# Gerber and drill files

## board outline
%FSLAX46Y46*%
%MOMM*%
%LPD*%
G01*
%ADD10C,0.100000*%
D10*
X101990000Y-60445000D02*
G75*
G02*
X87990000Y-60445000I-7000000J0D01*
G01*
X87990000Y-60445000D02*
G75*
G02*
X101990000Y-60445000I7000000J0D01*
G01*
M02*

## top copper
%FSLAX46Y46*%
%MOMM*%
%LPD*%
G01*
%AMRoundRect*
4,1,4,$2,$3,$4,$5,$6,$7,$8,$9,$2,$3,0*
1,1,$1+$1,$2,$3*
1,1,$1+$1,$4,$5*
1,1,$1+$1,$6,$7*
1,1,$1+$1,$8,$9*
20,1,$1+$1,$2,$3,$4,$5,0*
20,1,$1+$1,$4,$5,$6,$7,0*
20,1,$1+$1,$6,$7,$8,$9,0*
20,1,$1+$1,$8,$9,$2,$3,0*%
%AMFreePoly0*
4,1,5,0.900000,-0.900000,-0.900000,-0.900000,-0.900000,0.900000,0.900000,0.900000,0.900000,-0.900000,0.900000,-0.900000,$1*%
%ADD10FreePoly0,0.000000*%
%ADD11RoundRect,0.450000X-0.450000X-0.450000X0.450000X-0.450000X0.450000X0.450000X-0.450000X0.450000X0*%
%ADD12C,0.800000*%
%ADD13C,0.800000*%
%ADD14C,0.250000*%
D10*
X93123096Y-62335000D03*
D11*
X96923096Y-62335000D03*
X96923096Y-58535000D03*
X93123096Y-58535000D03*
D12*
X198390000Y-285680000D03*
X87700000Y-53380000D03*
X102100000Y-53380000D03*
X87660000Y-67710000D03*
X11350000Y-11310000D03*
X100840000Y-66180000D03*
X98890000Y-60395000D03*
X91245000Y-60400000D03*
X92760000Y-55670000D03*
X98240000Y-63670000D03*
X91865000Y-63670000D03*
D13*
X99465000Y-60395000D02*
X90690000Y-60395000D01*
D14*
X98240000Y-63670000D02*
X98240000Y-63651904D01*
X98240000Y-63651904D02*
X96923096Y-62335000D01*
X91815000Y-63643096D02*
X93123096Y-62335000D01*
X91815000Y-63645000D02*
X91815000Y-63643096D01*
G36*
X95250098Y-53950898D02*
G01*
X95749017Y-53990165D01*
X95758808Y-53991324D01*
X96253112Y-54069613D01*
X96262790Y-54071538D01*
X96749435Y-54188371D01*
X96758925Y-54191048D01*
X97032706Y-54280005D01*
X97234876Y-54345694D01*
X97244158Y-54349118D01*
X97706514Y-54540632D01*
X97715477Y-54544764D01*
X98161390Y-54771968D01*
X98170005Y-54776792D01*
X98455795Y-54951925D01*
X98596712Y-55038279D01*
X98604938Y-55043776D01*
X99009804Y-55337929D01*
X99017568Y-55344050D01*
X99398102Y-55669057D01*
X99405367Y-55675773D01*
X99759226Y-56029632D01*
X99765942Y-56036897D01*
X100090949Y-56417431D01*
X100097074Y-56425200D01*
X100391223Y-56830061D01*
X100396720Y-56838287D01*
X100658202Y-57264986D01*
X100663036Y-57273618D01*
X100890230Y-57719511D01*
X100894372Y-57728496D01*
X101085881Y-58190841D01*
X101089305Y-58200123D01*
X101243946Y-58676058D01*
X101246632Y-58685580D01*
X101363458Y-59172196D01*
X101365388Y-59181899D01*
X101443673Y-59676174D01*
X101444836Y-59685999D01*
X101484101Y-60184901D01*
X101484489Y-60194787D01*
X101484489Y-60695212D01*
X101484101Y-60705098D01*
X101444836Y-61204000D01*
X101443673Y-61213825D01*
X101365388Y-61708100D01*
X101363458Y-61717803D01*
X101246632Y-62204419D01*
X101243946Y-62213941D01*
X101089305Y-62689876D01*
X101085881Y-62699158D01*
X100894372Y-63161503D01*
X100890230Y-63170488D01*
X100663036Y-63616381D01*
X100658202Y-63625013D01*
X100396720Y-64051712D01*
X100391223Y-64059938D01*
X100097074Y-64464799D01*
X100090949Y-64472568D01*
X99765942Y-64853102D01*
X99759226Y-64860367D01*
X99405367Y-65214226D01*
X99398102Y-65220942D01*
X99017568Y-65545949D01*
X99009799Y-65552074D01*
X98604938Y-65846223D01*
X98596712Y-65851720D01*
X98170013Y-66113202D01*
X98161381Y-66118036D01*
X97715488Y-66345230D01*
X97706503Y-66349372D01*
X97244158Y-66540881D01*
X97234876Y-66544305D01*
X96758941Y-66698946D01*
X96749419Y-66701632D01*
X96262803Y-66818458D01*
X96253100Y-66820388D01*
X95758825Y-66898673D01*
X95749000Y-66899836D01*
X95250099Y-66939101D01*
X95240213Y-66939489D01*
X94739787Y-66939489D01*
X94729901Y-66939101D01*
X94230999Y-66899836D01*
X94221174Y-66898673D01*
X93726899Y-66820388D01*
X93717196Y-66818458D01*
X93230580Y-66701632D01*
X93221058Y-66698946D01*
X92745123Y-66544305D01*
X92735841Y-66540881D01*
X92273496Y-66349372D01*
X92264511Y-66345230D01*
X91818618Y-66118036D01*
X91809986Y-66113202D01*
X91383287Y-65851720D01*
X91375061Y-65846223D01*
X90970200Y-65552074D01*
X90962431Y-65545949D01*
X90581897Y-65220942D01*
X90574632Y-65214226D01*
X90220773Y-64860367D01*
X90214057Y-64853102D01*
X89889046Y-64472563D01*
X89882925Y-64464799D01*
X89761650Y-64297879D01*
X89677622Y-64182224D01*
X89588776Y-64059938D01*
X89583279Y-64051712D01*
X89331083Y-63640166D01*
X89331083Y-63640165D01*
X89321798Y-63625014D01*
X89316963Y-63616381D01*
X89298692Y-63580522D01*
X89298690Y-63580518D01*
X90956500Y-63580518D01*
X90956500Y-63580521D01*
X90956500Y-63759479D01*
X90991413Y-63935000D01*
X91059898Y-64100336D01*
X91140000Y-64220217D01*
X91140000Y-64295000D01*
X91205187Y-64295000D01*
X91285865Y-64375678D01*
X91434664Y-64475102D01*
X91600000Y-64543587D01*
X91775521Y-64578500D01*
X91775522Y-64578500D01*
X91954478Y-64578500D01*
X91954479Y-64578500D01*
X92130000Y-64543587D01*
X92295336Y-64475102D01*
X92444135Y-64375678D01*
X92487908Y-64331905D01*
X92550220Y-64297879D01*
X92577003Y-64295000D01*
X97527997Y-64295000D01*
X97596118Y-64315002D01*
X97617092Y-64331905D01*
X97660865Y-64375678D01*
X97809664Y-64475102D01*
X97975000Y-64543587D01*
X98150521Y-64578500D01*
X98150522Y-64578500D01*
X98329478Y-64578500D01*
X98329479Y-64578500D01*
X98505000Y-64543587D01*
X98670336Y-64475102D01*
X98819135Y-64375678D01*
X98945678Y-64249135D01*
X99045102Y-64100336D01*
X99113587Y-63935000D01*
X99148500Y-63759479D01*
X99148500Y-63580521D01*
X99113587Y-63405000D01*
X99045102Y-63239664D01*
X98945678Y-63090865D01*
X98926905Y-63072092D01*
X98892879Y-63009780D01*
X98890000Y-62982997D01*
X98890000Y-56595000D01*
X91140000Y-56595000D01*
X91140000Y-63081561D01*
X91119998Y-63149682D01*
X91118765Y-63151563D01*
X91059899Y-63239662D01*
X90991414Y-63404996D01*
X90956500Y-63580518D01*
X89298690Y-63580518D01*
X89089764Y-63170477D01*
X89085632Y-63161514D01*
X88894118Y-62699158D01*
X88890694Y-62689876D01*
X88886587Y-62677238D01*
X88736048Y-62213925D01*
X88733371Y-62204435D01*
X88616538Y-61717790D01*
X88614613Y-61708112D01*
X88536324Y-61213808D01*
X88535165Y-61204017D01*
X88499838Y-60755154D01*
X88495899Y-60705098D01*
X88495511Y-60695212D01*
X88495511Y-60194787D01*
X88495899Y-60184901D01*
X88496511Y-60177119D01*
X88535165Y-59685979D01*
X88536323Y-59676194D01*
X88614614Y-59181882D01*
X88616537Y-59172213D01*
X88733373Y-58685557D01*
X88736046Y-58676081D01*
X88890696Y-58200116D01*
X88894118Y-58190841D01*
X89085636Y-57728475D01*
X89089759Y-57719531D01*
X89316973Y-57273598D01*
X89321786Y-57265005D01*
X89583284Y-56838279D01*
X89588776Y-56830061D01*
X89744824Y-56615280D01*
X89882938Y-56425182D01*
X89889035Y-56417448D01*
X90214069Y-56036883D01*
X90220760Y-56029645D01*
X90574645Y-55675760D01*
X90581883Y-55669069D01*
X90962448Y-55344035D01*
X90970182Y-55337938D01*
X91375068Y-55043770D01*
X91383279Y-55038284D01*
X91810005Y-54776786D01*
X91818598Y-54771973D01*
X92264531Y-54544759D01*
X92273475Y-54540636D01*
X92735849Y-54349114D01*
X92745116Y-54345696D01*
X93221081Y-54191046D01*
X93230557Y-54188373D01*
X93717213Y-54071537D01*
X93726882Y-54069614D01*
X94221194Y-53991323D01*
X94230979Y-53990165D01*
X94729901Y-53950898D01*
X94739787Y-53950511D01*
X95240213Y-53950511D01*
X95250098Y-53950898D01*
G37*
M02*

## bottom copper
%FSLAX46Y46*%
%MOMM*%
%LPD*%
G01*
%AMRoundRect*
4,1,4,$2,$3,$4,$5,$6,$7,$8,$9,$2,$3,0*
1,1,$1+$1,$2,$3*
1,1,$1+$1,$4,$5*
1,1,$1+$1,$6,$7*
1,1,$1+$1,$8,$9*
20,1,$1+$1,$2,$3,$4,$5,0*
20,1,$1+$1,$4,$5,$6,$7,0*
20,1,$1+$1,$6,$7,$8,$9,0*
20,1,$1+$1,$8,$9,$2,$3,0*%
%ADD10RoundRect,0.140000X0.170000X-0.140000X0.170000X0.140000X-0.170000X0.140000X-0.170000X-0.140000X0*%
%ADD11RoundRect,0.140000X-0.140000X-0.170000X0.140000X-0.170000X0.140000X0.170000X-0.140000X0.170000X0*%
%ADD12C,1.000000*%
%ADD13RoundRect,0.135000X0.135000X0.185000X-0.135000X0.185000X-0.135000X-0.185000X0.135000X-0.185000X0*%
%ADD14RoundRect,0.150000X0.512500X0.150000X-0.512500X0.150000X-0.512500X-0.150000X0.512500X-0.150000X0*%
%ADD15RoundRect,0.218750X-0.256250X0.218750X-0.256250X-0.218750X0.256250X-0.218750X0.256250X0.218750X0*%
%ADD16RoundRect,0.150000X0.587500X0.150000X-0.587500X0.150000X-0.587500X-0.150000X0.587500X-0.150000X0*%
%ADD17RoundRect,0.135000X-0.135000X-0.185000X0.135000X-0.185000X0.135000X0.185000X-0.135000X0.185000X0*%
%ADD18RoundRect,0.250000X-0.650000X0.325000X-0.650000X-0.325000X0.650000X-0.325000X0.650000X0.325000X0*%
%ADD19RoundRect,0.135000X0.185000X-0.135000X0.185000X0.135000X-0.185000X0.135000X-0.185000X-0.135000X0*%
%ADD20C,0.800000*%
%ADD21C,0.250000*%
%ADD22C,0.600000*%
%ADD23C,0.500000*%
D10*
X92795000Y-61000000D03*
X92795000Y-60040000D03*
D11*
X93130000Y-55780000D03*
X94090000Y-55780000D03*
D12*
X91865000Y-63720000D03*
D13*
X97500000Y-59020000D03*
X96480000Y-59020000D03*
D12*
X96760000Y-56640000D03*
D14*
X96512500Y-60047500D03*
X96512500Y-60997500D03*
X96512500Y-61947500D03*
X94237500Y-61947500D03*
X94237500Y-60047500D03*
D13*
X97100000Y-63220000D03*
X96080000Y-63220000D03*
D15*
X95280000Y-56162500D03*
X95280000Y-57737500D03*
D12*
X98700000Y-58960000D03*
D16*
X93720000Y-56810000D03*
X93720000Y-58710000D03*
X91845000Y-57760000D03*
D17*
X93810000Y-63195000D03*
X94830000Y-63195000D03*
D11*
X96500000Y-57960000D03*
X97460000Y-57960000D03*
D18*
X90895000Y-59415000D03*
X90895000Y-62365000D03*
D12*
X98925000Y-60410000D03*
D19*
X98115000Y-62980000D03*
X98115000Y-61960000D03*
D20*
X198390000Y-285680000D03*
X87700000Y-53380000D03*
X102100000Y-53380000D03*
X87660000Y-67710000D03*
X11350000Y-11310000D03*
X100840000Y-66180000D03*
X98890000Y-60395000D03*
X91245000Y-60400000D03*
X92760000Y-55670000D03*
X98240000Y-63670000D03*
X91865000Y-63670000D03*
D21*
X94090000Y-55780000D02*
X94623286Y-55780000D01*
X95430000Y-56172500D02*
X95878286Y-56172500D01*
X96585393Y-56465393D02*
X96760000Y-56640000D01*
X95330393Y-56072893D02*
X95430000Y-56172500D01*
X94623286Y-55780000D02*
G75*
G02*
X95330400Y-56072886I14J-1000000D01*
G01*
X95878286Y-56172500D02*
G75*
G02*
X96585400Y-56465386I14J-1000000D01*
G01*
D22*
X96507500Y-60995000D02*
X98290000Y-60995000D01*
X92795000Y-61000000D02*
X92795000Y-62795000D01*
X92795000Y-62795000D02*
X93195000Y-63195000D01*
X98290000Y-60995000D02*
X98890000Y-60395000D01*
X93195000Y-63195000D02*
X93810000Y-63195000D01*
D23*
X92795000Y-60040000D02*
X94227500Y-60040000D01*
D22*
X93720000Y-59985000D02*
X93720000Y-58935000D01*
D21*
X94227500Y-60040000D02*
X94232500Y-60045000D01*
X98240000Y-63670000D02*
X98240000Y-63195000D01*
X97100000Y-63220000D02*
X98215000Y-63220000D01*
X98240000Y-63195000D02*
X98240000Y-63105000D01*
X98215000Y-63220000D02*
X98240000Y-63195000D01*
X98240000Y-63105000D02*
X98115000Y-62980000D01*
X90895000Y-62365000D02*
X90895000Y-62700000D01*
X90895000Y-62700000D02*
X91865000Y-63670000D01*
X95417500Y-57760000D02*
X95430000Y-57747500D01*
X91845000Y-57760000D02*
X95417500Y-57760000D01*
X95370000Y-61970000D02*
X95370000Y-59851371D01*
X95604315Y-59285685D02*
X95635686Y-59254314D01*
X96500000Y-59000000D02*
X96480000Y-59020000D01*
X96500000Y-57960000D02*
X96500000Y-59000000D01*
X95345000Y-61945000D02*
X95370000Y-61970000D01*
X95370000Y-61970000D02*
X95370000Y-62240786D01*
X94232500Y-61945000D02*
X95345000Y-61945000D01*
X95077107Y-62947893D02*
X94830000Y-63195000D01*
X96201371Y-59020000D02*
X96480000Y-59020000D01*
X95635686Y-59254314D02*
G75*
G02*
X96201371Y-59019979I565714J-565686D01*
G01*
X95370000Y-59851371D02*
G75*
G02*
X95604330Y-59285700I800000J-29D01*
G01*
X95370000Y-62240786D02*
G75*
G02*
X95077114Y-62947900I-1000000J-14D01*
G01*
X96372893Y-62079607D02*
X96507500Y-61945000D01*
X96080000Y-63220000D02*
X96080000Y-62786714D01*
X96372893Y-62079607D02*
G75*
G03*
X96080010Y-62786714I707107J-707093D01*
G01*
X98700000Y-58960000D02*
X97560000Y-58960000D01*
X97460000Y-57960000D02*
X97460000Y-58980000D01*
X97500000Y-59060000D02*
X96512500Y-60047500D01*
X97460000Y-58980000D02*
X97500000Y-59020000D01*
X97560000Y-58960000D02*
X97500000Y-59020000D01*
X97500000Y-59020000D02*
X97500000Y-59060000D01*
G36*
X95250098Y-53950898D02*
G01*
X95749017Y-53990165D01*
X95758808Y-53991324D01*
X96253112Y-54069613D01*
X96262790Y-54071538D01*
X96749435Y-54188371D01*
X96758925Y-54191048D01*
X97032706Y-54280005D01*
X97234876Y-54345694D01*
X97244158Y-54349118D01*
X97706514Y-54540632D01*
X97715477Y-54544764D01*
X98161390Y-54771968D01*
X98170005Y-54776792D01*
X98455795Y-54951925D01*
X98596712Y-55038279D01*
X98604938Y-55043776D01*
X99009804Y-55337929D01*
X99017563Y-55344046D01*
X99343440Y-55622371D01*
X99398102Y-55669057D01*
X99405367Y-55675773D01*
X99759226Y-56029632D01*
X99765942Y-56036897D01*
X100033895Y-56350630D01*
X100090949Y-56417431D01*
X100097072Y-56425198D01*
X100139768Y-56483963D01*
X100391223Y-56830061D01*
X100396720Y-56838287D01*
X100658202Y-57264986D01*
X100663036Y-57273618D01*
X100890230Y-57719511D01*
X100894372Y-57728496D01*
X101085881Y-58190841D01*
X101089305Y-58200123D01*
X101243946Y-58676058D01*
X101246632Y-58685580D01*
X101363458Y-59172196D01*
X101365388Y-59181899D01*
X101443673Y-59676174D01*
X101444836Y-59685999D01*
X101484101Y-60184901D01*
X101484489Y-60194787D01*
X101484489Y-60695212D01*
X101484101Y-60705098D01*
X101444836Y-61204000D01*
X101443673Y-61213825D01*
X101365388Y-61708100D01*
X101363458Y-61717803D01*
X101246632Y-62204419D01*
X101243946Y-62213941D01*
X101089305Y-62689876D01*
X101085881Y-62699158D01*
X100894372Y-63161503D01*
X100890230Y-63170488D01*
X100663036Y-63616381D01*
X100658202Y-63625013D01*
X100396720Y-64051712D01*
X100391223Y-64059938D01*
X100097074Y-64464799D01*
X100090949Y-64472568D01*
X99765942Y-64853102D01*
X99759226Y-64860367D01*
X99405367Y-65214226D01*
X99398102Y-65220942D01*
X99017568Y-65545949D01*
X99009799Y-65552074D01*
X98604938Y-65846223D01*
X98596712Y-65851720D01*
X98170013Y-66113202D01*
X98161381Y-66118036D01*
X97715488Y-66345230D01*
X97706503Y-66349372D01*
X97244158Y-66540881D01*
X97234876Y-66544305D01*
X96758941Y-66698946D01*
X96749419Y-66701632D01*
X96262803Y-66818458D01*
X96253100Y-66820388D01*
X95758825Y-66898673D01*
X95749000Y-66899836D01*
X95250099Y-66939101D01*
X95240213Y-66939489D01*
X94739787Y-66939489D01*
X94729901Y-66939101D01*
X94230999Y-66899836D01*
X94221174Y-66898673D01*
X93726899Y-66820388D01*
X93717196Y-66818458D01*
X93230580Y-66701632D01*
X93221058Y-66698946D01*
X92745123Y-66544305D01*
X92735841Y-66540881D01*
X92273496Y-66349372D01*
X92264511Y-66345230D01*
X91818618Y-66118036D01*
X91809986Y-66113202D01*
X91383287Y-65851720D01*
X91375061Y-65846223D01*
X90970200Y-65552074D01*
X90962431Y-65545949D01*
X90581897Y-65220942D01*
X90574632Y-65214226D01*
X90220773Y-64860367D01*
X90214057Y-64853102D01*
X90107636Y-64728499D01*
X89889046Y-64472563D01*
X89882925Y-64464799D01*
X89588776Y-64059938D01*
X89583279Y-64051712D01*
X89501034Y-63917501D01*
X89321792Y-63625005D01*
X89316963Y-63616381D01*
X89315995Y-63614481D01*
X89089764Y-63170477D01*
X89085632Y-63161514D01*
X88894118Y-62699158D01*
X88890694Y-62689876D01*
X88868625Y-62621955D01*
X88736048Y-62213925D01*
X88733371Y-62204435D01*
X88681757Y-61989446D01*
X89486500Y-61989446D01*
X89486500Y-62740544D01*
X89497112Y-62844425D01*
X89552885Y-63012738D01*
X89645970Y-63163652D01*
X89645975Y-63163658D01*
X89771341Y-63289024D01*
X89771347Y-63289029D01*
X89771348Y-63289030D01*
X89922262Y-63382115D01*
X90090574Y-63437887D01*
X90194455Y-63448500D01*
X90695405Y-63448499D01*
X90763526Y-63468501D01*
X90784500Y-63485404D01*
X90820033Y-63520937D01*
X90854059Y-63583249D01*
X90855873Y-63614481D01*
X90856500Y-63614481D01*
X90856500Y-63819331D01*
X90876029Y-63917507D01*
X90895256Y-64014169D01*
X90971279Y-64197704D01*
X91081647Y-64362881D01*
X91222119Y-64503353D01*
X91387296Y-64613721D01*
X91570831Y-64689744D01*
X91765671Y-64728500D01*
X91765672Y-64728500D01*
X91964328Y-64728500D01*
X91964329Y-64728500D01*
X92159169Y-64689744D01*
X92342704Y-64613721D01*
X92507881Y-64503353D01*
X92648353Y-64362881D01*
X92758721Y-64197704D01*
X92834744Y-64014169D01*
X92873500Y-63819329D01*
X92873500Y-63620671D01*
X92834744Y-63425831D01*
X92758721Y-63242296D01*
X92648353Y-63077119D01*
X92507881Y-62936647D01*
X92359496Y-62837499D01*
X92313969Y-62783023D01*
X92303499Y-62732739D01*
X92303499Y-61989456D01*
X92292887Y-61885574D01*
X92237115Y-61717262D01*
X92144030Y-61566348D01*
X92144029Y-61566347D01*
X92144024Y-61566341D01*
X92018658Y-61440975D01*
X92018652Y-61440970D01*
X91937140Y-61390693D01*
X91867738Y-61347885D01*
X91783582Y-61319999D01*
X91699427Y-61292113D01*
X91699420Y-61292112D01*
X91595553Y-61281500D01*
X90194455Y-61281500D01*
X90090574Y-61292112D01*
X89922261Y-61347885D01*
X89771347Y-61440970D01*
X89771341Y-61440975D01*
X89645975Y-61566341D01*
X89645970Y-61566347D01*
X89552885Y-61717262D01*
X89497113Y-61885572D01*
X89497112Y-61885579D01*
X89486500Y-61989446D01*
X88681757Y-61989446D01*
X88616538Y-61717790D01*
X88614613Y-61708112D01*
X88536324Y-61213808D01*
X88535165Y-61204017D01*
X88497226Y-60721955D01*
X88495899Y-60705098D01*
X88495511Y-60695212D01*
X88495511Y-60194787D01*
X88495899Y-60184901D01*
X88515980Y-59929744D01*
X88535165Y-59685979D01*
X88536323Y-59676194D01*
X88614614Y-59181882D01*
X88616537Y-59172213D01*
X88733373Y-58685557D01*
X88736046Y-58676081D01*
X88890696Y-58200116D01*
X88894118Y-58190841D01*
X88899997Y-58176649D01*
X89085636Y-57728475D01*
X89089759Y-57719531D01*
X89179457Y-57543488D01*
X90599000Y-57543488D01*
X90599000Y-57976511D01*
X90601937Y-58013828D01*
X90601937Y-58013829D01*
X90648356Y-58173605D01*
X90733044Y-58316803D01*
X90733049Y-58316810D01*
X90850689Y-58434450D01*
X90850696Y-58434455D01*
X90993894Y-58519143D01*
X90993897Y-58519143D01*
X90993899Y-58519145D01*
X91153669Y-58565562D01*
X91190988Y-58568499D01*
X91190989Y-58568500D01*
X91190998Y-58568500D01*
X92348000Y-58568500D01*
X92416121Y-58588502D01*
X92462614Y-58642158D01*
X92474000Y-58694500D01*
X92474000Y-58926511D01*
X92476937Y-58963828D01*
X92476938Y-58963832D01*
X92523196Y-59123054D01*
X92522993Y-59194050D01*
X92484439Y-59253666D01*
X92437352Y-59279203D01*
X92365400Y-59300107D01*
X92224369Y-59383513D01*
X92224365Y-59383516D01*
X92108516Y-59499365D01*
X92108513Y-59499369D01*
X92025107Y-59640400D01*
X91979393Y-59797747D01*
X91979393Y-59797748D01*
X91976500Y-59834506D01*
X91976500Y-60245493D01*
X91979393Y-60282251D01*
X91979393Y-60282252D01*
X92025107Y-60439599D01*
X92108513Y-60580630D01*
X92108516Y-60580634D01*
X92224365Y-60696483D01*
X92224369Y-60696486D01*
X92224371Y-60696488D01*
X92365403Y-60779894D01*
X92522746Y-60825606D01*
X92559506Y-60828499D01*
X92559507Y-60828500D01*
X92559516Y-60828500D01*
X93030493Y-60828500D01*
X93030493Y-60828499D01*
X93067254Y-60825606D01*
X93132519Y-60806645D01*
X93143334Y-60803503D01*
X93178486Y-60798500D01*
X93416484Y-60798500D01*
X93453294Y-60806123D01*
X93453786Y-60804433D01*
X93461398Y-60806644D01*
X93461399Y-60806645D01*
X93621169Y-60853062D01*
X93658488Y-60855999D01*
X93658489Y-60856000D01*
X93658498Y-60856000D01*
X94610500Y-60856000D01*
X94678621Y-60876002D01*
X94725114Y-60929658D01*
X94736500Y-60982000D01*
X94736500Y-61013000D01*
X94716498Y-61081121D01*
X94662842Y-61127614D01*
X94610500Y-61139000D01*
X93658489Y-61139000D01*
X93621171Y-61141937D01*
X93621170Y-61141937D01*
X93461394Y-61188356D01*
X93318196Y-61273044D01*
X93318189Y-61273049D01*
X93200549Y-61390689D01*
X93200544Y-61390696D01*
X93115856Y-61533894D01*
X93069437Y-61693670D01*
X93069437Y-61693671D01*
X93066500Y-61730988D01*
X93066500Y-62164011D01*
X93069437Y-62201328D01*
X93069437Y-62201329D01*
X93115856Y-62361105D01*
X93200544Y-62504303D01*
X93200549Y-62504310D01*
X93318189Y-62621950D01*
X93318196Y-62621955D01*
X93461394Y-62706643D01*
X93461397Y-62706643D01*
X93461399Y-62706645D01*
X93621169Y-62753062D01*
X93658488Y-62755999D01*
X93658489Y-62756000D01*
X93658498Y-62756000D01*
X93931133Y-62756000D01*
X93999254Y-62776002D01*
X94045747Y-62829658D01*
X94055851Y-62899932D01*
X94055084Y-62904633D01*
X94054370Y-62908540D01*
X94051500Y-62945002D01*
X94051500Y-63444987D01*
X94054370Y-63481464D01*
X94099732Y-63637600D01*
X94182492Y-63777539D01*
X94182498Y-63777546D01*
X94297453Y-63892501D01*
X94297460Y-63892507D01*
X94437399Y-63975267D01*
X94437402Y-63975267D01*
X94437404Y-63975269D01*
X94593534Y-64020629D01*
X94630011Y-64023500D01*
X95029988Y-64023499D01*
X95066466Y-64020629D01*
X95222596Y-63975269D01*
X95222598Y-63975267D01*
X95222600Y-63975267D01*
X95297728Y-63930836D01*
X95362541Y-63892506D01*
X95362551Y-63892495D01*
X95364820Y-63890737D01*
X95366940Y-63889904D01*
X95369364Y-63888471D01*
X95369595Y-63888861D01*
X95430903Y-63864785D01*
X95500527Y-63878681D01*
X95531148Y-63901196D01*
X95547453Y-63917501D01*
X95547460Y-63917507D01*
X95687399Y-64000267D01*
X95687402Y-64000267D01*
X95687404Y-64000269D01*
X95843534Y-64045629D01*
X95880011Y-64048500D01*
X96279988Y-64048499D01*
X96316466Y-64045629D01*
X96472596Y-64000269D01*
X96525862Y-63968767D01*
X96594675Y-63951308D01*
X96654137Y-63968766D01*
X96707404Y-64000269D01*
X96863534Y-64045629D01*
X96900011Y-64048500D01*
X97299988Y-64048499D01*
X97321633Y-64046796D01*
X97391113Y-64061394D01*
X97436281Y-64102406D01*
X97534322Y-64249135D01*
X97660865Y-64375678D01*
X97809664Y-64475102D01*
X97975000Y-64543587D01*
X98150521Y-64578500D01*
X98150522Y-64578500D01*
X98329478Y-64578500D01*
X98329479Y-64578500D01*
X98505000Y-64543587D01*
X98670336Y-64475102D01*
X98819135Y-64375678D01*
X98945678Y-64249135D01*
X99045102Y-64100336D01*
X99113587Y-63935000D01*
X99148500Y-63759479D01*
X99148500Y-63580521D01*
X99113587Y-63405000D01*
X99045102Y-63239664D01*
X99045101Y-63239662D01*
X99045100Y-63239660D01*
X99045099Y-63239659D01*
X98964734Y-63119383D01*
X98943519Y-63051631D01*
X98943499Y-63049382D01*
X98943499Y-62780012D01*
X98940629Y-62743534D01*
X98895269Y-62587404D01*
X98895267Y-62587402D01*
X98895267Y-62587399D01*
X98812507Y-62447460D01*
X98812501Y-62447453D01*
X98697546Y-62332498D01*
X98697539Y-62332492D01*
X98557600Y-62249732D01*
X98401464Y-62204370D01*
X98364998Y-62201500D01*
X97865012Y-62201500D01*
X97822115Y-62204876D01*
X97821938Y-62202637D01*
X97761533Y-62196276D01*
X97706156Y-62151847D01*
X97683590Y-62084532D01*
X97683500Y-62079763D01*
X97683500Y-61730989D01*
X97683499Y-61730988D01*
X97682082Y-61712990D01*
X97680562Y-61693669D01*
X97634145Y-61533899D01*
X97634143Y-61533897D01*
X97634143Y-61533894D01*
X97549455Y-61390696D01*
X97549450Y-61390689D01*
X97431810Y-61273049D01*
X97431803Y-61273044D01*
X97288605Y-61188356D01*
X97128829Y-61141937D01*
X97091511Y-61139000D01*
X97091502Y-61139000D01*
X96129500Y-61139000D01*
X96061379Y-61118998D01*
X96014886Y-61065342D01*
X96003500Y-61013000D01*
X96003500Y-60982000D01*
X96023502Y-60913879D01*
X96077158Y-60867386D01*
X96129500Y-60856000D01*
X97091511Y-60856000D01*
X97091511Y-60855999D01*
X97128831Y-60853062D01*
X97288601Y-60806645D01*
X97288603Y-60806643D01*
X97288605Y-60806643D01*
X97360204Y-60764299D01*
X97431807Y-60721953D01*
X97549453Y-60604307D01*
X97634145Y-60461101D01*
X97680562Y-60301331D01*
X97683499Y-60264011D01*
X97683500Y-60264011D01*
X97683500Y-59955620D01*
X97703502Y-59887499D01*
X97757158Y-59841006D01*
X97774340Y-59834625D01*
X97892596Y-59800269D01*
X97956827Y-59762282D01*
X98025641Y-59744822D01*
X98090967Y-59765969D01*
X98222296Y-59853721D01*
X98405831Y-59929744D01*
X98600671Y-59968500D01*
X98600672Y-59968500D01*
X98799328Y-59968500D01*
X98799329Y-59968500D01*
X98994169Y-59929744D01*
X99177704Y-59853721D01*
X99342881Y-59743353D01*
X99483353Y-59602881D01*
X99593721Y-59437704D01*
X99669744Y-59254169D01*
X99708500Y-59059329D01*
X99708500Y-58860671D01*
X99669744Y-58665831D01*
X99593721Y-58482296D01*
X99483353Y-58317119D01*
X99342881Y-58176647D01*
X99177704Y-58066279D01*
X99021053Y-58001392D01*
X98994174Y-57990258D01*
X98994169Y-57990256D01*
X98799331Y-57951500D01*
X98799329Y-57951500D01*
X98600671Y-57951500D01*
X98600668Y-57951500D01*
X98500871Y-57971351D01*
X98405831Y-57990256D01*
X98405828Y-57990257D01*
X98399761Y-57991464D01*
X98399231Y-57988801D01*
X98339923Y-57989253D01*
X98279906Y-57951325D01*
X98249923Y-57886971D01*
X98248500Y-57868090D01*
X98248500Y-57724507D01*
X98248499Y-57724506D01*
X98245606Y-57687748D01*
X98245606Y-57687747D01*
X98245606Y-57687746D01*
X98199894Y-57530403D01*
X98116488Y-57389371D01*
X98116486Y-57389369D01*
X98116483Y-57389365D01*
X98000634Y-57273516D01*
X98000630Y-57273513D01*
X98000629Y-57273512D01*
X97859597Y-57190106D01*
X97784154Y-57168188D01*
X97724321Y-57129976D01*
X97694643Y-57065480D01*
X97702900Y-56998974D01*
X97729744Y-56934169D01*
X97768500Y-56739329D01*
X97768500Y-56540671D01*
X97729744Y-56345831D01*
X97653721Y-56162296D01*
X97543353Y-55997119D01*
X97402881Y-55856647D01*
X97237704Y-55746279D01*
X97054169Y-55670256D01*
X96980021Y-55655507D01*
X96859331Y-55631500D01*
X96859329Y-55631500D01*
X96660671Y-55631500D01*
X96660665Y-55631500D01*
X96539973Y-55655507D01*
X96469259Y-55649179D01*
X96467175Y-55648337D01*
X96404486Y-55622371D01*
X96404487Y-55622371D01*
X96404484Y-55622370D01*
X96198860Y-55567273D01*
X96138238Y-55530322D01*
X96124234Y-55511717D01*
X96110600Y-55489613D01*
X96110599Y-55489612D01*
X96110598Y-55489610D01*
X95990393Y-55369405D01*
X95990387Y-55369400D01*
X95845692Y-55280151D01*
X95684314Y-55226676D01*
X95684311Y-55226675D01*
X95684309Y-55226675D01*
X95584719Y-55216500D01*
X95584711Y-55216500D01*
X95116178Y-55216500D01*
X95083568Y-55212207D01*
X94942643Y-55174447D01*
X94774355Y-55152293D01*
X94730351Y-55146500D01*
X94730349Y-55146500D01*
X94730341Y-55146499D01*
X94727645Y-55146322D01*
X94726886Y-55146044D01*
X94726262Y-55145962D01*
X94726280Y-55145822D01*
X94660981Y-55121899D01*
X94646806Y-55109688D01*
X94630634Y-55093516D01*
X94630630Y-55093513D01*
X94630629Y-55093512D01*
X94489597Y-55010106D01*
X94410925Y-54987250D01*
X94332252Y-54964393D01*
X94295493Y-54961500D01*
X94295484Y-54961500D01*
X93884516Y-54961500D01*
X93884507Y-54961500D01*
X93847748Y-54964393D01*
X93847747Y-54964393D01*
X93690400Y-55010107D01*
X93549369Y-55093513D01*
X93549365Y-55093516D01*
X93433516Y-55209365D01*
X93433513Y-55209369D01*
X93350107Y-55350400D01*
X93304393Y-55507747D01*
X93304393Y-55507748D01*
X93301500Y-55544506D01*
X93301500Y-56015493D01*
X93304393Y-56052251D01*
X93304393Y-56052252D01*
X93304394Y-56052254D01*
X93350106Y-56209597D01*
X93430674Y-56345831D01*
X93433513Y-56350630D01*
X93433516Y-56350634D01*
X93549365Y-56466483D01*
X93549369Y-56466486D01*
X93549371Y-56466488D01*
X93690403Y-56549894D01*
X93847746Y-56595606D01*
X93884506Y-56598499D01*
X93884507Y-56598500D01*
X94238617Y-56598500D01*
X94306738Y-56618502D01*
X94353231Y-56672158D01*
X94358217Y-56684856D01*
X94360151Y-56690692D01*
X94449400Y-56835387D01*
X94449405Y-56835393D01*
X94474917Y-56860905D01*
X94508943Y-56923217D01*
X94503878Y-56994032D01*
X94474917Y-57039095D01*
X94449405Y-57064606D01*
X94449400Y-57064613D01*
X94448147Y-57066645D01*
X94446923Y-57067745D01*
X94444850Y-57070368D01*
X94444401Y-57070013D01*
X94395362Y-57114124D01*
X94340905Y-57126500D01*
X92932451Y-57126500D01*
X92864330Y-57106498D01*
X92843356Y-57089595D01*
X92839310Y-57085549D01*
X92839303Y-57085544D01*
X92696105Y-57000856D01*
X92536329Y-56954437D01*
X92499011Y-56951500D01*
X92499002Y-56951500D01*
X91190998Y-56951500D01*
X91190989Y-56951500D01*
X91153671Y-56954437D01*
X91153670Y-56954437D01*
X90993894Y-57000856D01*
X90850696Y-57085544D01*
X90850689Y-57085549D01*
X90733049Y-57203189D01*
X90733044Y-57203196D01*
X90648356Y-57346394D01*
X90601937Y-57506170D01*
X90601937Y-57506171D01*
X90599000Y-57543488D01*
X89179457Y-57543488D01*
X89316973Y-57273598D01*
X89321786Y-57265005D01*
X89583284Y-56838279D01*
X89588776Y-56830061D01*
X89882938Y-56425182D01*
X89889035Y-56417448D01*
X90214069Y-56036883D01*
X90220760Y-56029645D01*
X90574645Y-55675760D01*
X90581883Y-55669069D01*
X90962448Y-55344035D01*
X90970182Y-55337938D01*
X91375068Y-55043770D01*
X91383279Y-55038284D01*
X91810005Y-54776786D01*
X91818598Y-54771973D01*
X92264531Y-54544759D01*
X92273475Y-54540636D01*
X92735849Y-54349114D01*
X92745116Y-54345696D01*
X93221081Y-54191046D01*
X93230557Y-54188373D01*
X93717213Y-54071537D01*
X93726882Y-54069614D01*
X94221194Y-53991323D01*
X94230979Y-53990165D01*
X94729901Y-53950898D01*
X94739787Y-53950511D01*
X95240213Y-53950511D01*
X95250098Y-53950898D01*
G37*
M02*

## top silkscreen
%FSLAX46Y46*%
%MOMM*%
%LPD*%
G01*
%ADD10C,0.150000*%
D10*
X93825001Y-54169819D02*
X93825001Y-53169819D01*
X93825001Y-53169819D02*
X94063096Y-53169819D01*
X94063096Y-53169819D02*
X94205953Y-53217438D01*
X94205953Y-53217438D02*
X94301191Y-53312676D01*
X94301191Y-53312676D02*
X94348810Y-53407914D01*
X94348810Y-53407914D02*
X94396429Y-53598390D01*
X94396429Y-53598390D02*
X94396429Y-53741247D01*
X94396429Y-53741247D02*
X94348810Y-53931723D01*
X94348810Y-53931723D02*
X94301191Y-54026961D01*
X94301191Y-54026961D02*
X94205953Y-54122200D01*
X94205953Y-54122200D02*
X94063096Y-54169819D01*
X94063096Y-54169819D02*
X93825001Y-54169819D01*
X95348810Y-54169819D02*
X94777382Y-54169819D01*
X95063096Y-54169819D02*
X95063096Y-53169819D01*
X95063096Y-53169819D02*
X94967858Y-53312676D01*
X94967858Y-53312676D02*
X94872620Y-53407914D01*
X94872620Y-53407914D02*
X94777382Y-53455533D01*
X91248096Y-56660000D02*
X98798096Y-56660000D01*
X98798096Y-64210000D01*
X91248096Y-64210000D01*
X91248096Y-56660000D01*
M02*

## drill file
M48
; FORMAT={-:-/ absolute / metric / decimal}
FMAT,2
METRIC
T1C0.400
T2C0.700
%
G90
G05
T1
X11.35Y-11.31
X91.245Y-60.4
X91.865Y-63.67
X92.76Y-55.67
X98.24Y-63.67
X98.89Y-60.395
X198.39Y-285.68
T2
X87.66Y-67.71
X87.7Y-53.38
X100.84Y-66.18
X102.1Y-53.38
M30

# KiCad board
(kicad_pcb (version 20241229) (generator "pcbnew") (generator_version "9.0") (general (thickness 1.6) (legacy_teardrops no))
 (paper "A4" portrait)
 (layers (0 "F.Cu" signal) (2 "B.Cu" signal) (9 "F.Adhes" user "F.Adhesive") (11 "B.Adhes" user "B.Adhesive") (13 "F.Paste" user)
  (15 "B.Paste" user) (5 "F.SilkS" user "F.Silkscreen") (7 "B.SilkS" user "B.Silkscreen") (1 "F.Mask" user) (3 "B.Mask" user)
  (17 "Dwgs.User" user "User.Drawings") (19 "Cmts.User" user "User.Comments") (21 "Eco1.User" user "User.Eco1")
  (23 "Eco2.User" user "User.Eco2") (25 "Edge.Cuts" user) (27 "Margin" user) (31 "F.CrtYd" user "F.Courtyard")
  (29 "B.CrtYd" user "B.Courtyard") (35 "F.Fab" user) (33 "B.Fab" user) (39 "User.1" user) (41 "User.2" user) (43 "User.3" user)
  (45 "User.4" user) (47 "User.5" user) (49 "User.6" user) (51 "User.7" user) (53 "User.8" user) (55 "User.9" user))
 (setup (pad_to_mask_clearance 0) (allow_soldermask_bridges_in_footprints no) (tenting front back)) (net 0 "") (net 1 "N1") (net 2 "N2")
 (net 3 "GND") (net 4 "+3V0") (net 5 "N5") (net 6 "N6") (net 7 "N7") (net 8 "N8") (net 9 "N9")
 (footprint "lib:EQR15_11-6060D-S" (layer "F.Cu") (at 95.023096 60.435)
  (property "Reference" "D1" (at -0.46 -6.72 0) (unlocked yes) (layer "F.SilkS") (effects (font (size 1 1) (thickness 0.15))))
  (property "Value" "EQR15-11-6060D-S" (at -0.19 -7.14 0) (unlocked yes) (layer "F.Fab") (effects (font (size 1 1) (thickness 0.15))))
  (fp_rect (start -3.775 -3.775) (end 3.775 3.775) (stroke (width 0.15) (type solid)) (fill no) (layer "F.SilkS"))
  (pad "1" smd custom (at -1.9 1.9) (size 1.8 1.8) (layers "F.Cu" "F.Mask" "F.Paste") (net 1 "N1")
   (options (clearance outline) (anchor rect)) (primitives))
  (pad "2" smd roundrect (at 1.9 1.9) (size 1.8 1.8) (layers "F.Cu" "F.Mask" "F.Paste") (roundrect_rratio 0.25) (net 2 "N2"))
  (pad "3" smd roundrect (at 1.9 -1.9) (size 1.8 1.8) (layers "F.Cu" "F.Mask" "F.Paste") (roundrect_rratio 0.25))
  (pad "4" smd roundrect (at -1.9 -1.9) (size 1.8 1.8) (layers "F.Cu" "F.Mask" "F.Paste") (roundrect_rratio 0.25)))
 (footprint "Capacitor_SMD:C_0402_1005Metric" (layer "B.Cu") (at 92.795 60.52 90)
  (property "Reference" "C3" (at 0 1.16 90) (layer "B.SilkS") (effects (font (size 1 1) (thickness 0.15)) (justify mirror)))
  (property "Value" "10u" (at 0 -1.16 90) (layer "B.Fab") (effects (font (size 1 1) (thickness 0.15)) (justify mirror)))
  (pad "1" smd roundrect (at -0.48 0 90) (size 0.56 0.62) (layers "B.Cu" "B.Mask" "B.Paste") (roundrect_rratio 0.25) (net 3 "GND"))
  (pad "2" smd roundrect (at 0.48 0 90) (size 0.56 0.62) (layers "B.Cu" "B.Mask" "B.Paste") (roundrect_rratio 0.25) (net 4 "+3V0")))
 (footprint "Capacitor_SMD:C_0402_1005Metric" (layer "B.Cu") (at 93.61 55.78)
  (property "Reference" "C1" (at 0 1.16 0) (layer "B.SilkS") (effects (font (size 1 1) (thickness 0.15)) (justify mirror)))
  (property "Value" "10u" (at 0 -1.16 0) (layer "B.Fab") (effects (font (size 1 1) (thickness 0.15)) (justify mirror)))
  (pad "1" smd roundrect (at -0.48 0) (size 0.56 0.62) (layers "B.Cu" "B.Mask" "B.Paste") (roundrect_rratio 0.25) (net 3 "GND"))
  (pad "2" smd roundrect (at 0.48 0) (size 0.56 0.62) (layers "B.Cu" "B.Mask" "B.Paste") (roundrect_rratio 0.25) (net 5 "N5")))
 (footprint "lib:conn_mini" (layer "B.Cu") (at 91.865 63.72 180)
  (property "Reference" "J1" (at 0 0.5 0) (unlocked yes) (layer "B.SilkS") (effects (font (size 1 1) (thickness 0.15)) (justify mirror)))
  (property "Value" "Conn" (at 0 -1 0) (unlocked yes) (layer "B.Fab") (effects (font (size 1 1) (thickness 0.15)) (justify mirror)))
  (pad "1" smd circle (at 0 0 180) (size 1 1) (layers "B.Cu" "B.Mask" "B.Paste") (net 1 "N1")))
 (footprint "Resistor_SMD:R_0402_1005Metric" (layer "B.Cu") (at 96.99 59.02 180)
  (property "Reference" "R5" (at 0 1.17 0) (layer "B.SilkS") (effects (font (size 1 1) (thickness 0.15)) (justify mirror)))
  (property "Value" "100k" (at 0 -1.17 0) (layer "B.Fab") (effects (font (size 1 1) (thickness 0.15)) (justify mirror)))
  (pad "1" smd roundrect (at -0.51 0 180) (size 0.54 0.64) (layers "B.Cu" "B.Mask" "B.Paste") (roundrect_rratio 0.25) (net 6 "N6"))
  (pad "2" smd roundrect (at 0.51 0 180) (size 0.54 0.64) (layers "B.Cu" "B.Mask" "B.Paste") (roundrect_rratio 0.25) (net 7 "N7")))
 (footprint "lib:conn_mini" (layer "B.Cu") (at 96.76 56.64 180)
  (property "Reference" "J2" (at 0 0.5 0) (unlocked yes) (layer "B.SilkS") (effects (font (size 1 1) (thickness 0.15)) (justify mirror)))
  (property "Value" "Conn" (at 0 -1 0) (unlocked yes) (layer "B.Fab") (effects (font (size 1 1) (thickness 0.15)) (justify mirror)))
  (pad "1" smd circle (at 0 0 180) (size 1 1) (layers "B.Cu" "B.Mask" "B.Paste") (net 5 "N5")))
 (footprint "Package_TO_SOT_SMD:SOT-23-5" (layer "B.Cu") (at 95.375 60.9975 180)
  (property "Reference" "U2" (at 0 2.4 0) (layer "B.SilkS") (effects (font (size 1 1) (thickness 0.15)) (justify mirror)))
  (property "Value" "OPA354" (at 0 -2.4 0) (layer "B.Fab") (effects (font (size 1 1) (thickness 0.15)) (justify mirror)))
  (pad "1" smd roundrect (at -1.1375 0.95 180) (size 1.325 0.6) (layers "B.Cu" "B.Mask" "B.Paste") (roundrect_rratio 0.25) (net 6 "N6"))
  (pad "2" smd roundrect (at -1.1375 0 180) (size 1.325 0.6) (layers "B.Cu" "B.Mask" "B.Paste") (roundrect_rratio 0.25) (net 3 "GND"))
  (pad "3" smd roundrect (at -1.1375 -0.95 180) (size 1.325 0.6) (layers "B.Cu" "B.Mask" "B.Paste") (roundrect_rratio 0.25) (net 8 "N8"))
  (pad "4" smd roundrect (at 1.1375 -0.95 180) (size 1.325 0.6) (layers "B.Cu" "B.Mask" "B.Paste") (roundrect_rratio 0.25) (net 7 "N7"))
  (pad "5" smd roundrect (at 1.1375 0.95 180) (size 1.325 0.6) (layers "B.Cu" "B.Mask" "B.Paste") (roundrect_rratio 0.25) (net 4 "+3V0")))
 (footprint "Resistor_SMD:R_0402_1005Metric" (layer "B.Cu") (at 96.59 63.22 180)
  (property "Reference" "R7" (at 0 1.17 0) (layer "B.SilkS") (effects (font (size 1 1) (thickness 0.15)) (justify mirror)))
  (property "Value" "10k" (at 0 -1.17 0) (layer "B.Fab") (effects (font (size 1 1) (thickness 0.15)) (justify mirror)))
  (pad "1" smd roundrect (at -0.51 0 180) (size 0.54 0.64) (layers "B.Cu" "B.Mask" "B.Paste") (roundrect_rratio 0.25) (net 2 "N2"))
  (pad "2" smd roundrect (at 0.51 0 180) (size 0.54 0.64) (layers "B.Cu" "B.Mask" "B.Paste") (roundrect_rratio 0.25) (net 8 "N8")))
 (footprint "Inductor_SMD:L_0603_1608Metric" (layer "B.Cu") (at 95.28 56.95 -90)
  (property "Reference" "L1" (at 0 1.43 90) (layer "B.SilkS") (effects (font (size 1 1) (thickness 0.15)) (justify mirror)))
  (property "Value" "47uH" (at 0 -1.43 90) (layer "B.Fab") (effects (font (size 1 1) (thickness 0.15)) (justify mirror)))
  (pad "1" smd roundrect (at -0.7875 0 270) (size 0.875 0.95) (layers "B.Cu" "B.Mask" "B.Paste") (roundrect_rratio 0.25) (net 5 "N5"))
  (pad "2" smd roundrect (at 0.7875 0 270) (size 0.875 0.95) (layers "B.Cu" "B.Mask" "B.Paste") (roundrect_rratio 0.25) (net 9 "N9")))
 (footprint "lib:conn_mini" (layer "B.Cu") (at 98.7 58.96 180)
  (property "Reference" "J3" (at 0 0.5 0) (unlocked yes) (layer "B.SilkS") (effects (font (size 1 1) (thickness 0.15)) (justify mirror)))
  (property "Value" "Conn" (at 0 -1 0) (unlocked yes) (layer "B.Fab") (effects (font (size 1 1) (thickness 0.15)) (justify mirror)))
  (pad "1" smd circle (at 0 0 180) (size 1 1) (layers "B.Cu" "B.Mask" "B.Paste") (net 6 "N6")))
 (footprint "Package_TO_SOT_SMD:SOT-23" (layer "B.Cu") (at 92.7825 57.76 180)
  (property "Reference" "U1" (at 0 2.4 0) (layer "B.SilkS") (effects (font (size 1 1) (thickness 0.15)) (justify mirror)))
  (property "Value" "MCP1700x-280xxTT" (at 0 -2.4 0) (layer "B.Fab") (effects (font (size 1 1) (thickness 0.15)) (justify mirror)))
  (pad "1" smd roundrect (at -0.9375 0.95 180) (size 1.475 0.6) (layers "B.Cu" "B.Mask" "B.Paste") (roundrect_rratio 0.25) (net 3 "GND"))
  (pad "2" smd roundrect (at -0.9375 -0.95 180) (size 1.475 0.6) (layers "B.Cu" "B.Mask" "B.Paste") (roundrect_rratio 0.25) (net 4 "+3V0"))
  (pad "3" smd roundrect (at 0.9375 0 180) (size 1.475 0.6) (layers "B.Cu" "B.Mask" "B.Paste") (roundrect_rratio 0.25) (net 9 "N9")))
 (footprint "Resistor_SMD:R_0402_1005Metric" (layer "B.Cu") (at 94.32 63.195)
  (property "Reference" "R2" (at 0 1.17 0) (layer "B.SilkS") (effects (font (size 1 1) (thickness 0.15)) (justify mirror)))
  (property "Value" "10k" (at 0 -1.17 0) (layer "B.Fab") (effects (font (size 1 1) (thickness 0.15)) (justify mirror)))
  (pad "1" smd roundrect (at -0.51 0) (size 0.54 0.64) (layers "B.Cu" "B.Mask" "B.Paste") (roundrect_rratio 0.25) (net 3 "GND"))
  (pad "2" smd roundrect (at 0.51 0) (size 0.54 0.64) (layers "B.Cu" "B.Mask" "B.Paste") (roundrect_rratio 0.25) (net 7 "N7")))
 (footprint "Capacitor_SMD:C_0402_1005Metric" (layer "B.Cu") (at 96.98 57.96)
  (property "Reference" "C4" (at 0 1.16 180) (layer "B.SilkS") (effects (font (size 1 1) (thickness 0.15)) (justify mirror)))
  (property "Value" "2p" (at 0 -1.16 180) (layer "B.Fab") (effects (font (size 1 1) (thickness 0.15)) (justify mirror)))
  (pad "1" smd roundrect (at -0.48 0) (size 0.56 0.62) (layers "B.Cu" "B.Mask" "B.Paste") (roundrect_rratio 0.25) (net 7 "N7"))
  (pad "2" smd roundrect (at 0.48 0) (size 0.56 0.62) (layers "B.Cu" "B.Mask" "B.Paste") (roundrect_rratio 0.25) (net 6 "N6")))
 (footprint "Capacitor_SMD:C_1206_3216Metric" (layer "B.Cu") (at 90.895 60.89 -90)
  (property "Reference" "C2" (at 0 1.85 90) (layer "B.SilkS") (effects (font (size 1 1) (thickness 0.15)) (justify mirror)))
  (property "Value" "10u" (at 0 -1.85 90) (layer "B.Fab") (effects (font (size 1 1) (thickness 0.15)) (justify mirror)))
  (pad "1" smd roundrect (at -1.475 0 270) (size 1.15 1.8) (layers "B.Cu" "B.Mask" "B.Paste") (roundrect_rratio 0.217391) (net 3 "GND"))
  (pad "2" smd roundrect (at 1.475 0 270) (size 1.15 1.8) (layers "B.Cu" "B.Mask" "B.Paste") (roundrect_rratio 0.217391) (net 1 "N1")))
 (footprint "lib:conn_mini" (layer "B.Cu") (at 98.925 60.41 180)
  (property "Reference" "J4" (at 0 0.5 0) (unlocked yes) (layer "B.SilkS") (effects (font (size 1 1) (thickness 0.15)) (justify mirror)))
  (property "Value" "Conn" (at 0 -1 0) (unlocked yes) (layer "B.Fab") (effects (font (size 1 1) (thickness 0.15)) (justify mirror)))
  (pad "1" smd circle (at 0 0 180) (size 1 1) (layers "B.Cu" "B.Mask" "B.Paste") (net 3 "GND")))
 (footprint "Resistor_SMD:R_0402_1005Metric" (layer "B.Cu") (at 98.115 62.47 90)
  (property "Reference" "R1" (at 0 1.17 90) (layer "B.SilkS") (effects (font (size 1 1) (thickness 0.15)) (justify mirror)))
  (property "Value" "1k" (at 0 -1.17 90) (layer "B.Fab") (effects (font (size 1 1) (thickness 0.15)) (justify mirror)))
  (pad "1" smd roundrect (at -0.51 0 90) (size 0.54 0.64) (layers "B.Cu" "B.Mask" "B.Paste") (roundrect_rratio 0.25) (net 2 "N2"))
  (pad "2" smd roundrect (at 0.51 0 90) (size 0.54 0.64) (layers "B.Cu" "B.Mask" "B.Paste") (roundrect_rratio 0.25) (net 3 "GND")))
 (gr_circle (center 94.99 60.445) (end 101.99 60.445) (stroke (width 0.1) (type solid)) (fill no) (layer "Edge.Cuts"))
 (via (at 198.39 285.68) (size 0.8) (drill 0.4) (layers "F.Cu" "B.Cu") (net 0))
 (via (at 87.7 53.38) (size 0.8) (drill 0.7) (layers "F.Cu" "B.Cu") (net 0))
 (via (at 102.1 53.38) (size 0.8) (drill 0.7) (layers "F.Cu" "B.Cu") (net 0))
 (via (at 87.66 67.71) (size 0.8) (drill 0.7) (layers "F.Cu" "B.Cu") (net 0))
 (via (at 11.35 11.31) (size 0.8) (drill 0.4) (layers "F.Cu" "B.Cu") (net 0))
 (via (at 100.84 66.18) (size 0.8) (drill 0.7) (layers "F.Cu" "B.Cu") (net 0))
 (segment (start 94.09 55.78) (end 94.623286 55.78) (width 0.25) (layer "B.Cu") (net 5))
 (segment (start 95.43 56.1725) (end 95.878286 56.1725) (width 0.25) (layer "B.Cu") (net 5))
 (segment (start 96.585393 56.465393) (end 96.76 56.64) (width 0.25) (layer "B.Cu") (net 5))
 (segment (start 95.330393 56.072893) (end 95.43 56.1725) (width 0.25) (layer "B.Cu") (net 5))
 (arc (start 94.623286 55.78) (mid 95.005969 55.85612) (end 95.330393 56.072893) (width 0.25) (layer "B.Cu") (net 5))
 (arc (start 95.878286 56.1725) (mid 96.260969 56.24862) (end 96.585393 56.465393) (width 0.25) (layer "B.Cu") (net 5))
 (segment (start 99.465 60.395) (end 90.69 60.395) (width 0.8) (layer "F.Cu") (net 3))
 (via (at 98.89 60.395) (size 0.8) (drill 0.4) (layers "F.Cu" "B.Cu") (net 3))
 (via (at 91.245 60.4) (size 0.8) (drill 0.4) (layers "F.Cu" "B.Cu") (free yes) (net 3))
 (via (at 92.76 55.67) (size 0.8) (drill 0.4) (layers "F.Cu" "B.Cu") (free yes) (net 3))
 (segment (start 96.5075 60.995) (end 98.29 60.995) (width 0.6) (layer "B.Cu") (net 3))
 (segment (start 92.795 61) (end 92.795 62.795) (width 0.6) (layer "B.Cu") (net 3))
 (segment (start 92.795 62.795) (end 93.195 63.195) (width 0.6) (layer "B.Cu") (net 3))
 (segment (start 98.29 60.995) (end 98.89 60.395) (width 0.6) (layer "B.Cu") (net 3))
 (segment (start 93.195 63.195) (end 93.81 63.195) (width 0.6) (layer "B.Cu") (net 3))
 (segment (start 92.795 60.04) (end 94.2275 60.04) (width 0.5) (layer "B.Cu") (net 4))
 (segment (start 93.72 59.985) (end 93.72 58.935) (width 0.6) (layer "B.Cu") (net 4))
 (segment (start 94.2275 60.04) (end 94.2325 60.045) (width 0.25) (layer "B.Cu") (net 4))
 (segment (start 98.24 63.67) (end 98.24 63.651904) (width 0.25) (layer "F.Cu") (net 2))
 (segment (start 98.24 63.651904) (end 96.923096 62.335) (width 0.25) (layer "F.Cu") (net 2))
 (via (at 98.24 63.67) (size 0.8) (drill 0.4) (layers "F.Cu" "B.Cu") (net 2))
 (segment (start 98.24 63.67) (end 98.24 63.195) (width 0.25) (layer "B.Cu") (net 2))
 (segment (start 97.1 63.22) (end 98.215 63.22) (width 0.25) (layer "B.Cu") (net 2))
 (segment (start 98.24 63.195) (end 98.24 63.105) (width 0.25) (layer "B.Cu") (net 2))
 (segment (start 98.215 63.22) (end 98.24 63.195) (width 0.25) (layer "B.Cu") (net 2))
 (segment (start 98.24 63.105) (end 98.115 62.98) (width 0.25) (layer "B.Cu") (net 2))
 (segment (start 91.815 63.643096) (end 93.123096 62.335) (width 0.25) (layer "F.Cu") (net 1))
 (segment (start 91.815 63.645) (end 91.815 63.643096) (width 0.25) (layer "F.Cu") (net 1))
 (via (at 91.865 63.67) (size 0.8) (drill 0.4) (layers "F.Cu" "B.Cu") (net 1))
 (segment (start 90.895 62.365) (end 90.895 62.7) (width 0.25) (layer "B.Cu") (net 1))
 (segment (start 90.895 62.7) (end 91.865 63.67) (width 0.25) (layer "B.Cu") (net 1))
 (segment (start 95.4175 57.76) (end 95.43 57.7475) (width 0.25) (layer "B.Cu") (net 9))
 (segment (start 91.845 57.76) (end 95.4175 57.76) (width 0.25) (layer "B.Cu") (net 9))
 (segment (start 95.37 61.97) (end 95.37 59.851371) (width 0.25) (layer "B.Cu") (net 7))
 (segment (start 95.604315 59.285685) (end 95.635686 59.254314) (width 0.25) (layer "B.Cu") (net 7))
 (segment (start 96.5 59) (end 96.48 59.02) (width 0.25) (layer "B.Cu") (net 7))
 (segment (start 96.5 57.96) (end 96.5 59) (width 0.25) (layer "B.Cu") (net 7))
 (segment (start 95.345 61.945) (end 95.37 61.97) (width 0.25) (layer "B.Cu") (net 7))
 (segment (start 95.37 61.97) (end 95.37 62.240786) (width 0.25) (layer "B.Cu") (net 7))
 (segment (start 94.2325 61.945) (end 95.345 61.945) (width 0.25) (layer "B.Cu") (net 7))
 (segment (start 95.077107 62.947893) (end 94.83 63.195) (width 0.25) (layer "B.Cu") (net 7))
 (segment (start 96.201371 59.02) (end 96.48 59.02) (width 0.25) (layer "B.Cu") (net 7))
 (arc (start 95.635686 59.254314) (mid 95.895225 59.080896) (end 96.201371 59.02) (width 0.25) (layer "B.Cu") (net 7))
 (arc (start 95.37 59.851371) (mid 95.430897 59.545224) (end 95.604315 59.285685) (width 0.25) (layer "B.Cu") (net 7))
 (arc (start 95.37 62.240786) (mid 95.29388 62.623469) (end 95.077107 62.947893) (width 0.25) (layer "B.Cu") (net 7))
 (segment (start 96.372893 62.079607) (end 96.5075 61.945) (width 0.25) (layer "B.Cu") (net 8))
 (segment (start 96.08 63.22) (end 96.08 62.786714) (width 0.25) (layer "B.Cu") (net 8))
 (arc (start 96.372893 62.079607) (mid 96.15612 62.40403) (end 96.08 62.786714) (width 0.25) (layer "B.Cu") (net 8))
 (segment (start 98.7 58.96) (end 97.56 58.96) (width 0.25) (layer "B.Cu") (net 6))
 (segment (start 97.46 57.96) (end 97.46 58.98) (width 0.25) (layer "B.Cu") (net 6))
 (segment (start 97.5 59.06) (end 96.5125 60.0475) (width 0.25) (layer "B.Cu") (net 6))
 (segment (start 97.46 58.98) (end 97.5 59.02) (width 0.25) (layer "B.Cu") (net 6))
 (segment (start 97.56 58.96) (end 97.5 59.02) (width 0.25) (layer "B.Cu") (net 6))
 (segment (start 97.5 59.02) (end 97.5 59.06) (width 0.25) (layer "B.Cu") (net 6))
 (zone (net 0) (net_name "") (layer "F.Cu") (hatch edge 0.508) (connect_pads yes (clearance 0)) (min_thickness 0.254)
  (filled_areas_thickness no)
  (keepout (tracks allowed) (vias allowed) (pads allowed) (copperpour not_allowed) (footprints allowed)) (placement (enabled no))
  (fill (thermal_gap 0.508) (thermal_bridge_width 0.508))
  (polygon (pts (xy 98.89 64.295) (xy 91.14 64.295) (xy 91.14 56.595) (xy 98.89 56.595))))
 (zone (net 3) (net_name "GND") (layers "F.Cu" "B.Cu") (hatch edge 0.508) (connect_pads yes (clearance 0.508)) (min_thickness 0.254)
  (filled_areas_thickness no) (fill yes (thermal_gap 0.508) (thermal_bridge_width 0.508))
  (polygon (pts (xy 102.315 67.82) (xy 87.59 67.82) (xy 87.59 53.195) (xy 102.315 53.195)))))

